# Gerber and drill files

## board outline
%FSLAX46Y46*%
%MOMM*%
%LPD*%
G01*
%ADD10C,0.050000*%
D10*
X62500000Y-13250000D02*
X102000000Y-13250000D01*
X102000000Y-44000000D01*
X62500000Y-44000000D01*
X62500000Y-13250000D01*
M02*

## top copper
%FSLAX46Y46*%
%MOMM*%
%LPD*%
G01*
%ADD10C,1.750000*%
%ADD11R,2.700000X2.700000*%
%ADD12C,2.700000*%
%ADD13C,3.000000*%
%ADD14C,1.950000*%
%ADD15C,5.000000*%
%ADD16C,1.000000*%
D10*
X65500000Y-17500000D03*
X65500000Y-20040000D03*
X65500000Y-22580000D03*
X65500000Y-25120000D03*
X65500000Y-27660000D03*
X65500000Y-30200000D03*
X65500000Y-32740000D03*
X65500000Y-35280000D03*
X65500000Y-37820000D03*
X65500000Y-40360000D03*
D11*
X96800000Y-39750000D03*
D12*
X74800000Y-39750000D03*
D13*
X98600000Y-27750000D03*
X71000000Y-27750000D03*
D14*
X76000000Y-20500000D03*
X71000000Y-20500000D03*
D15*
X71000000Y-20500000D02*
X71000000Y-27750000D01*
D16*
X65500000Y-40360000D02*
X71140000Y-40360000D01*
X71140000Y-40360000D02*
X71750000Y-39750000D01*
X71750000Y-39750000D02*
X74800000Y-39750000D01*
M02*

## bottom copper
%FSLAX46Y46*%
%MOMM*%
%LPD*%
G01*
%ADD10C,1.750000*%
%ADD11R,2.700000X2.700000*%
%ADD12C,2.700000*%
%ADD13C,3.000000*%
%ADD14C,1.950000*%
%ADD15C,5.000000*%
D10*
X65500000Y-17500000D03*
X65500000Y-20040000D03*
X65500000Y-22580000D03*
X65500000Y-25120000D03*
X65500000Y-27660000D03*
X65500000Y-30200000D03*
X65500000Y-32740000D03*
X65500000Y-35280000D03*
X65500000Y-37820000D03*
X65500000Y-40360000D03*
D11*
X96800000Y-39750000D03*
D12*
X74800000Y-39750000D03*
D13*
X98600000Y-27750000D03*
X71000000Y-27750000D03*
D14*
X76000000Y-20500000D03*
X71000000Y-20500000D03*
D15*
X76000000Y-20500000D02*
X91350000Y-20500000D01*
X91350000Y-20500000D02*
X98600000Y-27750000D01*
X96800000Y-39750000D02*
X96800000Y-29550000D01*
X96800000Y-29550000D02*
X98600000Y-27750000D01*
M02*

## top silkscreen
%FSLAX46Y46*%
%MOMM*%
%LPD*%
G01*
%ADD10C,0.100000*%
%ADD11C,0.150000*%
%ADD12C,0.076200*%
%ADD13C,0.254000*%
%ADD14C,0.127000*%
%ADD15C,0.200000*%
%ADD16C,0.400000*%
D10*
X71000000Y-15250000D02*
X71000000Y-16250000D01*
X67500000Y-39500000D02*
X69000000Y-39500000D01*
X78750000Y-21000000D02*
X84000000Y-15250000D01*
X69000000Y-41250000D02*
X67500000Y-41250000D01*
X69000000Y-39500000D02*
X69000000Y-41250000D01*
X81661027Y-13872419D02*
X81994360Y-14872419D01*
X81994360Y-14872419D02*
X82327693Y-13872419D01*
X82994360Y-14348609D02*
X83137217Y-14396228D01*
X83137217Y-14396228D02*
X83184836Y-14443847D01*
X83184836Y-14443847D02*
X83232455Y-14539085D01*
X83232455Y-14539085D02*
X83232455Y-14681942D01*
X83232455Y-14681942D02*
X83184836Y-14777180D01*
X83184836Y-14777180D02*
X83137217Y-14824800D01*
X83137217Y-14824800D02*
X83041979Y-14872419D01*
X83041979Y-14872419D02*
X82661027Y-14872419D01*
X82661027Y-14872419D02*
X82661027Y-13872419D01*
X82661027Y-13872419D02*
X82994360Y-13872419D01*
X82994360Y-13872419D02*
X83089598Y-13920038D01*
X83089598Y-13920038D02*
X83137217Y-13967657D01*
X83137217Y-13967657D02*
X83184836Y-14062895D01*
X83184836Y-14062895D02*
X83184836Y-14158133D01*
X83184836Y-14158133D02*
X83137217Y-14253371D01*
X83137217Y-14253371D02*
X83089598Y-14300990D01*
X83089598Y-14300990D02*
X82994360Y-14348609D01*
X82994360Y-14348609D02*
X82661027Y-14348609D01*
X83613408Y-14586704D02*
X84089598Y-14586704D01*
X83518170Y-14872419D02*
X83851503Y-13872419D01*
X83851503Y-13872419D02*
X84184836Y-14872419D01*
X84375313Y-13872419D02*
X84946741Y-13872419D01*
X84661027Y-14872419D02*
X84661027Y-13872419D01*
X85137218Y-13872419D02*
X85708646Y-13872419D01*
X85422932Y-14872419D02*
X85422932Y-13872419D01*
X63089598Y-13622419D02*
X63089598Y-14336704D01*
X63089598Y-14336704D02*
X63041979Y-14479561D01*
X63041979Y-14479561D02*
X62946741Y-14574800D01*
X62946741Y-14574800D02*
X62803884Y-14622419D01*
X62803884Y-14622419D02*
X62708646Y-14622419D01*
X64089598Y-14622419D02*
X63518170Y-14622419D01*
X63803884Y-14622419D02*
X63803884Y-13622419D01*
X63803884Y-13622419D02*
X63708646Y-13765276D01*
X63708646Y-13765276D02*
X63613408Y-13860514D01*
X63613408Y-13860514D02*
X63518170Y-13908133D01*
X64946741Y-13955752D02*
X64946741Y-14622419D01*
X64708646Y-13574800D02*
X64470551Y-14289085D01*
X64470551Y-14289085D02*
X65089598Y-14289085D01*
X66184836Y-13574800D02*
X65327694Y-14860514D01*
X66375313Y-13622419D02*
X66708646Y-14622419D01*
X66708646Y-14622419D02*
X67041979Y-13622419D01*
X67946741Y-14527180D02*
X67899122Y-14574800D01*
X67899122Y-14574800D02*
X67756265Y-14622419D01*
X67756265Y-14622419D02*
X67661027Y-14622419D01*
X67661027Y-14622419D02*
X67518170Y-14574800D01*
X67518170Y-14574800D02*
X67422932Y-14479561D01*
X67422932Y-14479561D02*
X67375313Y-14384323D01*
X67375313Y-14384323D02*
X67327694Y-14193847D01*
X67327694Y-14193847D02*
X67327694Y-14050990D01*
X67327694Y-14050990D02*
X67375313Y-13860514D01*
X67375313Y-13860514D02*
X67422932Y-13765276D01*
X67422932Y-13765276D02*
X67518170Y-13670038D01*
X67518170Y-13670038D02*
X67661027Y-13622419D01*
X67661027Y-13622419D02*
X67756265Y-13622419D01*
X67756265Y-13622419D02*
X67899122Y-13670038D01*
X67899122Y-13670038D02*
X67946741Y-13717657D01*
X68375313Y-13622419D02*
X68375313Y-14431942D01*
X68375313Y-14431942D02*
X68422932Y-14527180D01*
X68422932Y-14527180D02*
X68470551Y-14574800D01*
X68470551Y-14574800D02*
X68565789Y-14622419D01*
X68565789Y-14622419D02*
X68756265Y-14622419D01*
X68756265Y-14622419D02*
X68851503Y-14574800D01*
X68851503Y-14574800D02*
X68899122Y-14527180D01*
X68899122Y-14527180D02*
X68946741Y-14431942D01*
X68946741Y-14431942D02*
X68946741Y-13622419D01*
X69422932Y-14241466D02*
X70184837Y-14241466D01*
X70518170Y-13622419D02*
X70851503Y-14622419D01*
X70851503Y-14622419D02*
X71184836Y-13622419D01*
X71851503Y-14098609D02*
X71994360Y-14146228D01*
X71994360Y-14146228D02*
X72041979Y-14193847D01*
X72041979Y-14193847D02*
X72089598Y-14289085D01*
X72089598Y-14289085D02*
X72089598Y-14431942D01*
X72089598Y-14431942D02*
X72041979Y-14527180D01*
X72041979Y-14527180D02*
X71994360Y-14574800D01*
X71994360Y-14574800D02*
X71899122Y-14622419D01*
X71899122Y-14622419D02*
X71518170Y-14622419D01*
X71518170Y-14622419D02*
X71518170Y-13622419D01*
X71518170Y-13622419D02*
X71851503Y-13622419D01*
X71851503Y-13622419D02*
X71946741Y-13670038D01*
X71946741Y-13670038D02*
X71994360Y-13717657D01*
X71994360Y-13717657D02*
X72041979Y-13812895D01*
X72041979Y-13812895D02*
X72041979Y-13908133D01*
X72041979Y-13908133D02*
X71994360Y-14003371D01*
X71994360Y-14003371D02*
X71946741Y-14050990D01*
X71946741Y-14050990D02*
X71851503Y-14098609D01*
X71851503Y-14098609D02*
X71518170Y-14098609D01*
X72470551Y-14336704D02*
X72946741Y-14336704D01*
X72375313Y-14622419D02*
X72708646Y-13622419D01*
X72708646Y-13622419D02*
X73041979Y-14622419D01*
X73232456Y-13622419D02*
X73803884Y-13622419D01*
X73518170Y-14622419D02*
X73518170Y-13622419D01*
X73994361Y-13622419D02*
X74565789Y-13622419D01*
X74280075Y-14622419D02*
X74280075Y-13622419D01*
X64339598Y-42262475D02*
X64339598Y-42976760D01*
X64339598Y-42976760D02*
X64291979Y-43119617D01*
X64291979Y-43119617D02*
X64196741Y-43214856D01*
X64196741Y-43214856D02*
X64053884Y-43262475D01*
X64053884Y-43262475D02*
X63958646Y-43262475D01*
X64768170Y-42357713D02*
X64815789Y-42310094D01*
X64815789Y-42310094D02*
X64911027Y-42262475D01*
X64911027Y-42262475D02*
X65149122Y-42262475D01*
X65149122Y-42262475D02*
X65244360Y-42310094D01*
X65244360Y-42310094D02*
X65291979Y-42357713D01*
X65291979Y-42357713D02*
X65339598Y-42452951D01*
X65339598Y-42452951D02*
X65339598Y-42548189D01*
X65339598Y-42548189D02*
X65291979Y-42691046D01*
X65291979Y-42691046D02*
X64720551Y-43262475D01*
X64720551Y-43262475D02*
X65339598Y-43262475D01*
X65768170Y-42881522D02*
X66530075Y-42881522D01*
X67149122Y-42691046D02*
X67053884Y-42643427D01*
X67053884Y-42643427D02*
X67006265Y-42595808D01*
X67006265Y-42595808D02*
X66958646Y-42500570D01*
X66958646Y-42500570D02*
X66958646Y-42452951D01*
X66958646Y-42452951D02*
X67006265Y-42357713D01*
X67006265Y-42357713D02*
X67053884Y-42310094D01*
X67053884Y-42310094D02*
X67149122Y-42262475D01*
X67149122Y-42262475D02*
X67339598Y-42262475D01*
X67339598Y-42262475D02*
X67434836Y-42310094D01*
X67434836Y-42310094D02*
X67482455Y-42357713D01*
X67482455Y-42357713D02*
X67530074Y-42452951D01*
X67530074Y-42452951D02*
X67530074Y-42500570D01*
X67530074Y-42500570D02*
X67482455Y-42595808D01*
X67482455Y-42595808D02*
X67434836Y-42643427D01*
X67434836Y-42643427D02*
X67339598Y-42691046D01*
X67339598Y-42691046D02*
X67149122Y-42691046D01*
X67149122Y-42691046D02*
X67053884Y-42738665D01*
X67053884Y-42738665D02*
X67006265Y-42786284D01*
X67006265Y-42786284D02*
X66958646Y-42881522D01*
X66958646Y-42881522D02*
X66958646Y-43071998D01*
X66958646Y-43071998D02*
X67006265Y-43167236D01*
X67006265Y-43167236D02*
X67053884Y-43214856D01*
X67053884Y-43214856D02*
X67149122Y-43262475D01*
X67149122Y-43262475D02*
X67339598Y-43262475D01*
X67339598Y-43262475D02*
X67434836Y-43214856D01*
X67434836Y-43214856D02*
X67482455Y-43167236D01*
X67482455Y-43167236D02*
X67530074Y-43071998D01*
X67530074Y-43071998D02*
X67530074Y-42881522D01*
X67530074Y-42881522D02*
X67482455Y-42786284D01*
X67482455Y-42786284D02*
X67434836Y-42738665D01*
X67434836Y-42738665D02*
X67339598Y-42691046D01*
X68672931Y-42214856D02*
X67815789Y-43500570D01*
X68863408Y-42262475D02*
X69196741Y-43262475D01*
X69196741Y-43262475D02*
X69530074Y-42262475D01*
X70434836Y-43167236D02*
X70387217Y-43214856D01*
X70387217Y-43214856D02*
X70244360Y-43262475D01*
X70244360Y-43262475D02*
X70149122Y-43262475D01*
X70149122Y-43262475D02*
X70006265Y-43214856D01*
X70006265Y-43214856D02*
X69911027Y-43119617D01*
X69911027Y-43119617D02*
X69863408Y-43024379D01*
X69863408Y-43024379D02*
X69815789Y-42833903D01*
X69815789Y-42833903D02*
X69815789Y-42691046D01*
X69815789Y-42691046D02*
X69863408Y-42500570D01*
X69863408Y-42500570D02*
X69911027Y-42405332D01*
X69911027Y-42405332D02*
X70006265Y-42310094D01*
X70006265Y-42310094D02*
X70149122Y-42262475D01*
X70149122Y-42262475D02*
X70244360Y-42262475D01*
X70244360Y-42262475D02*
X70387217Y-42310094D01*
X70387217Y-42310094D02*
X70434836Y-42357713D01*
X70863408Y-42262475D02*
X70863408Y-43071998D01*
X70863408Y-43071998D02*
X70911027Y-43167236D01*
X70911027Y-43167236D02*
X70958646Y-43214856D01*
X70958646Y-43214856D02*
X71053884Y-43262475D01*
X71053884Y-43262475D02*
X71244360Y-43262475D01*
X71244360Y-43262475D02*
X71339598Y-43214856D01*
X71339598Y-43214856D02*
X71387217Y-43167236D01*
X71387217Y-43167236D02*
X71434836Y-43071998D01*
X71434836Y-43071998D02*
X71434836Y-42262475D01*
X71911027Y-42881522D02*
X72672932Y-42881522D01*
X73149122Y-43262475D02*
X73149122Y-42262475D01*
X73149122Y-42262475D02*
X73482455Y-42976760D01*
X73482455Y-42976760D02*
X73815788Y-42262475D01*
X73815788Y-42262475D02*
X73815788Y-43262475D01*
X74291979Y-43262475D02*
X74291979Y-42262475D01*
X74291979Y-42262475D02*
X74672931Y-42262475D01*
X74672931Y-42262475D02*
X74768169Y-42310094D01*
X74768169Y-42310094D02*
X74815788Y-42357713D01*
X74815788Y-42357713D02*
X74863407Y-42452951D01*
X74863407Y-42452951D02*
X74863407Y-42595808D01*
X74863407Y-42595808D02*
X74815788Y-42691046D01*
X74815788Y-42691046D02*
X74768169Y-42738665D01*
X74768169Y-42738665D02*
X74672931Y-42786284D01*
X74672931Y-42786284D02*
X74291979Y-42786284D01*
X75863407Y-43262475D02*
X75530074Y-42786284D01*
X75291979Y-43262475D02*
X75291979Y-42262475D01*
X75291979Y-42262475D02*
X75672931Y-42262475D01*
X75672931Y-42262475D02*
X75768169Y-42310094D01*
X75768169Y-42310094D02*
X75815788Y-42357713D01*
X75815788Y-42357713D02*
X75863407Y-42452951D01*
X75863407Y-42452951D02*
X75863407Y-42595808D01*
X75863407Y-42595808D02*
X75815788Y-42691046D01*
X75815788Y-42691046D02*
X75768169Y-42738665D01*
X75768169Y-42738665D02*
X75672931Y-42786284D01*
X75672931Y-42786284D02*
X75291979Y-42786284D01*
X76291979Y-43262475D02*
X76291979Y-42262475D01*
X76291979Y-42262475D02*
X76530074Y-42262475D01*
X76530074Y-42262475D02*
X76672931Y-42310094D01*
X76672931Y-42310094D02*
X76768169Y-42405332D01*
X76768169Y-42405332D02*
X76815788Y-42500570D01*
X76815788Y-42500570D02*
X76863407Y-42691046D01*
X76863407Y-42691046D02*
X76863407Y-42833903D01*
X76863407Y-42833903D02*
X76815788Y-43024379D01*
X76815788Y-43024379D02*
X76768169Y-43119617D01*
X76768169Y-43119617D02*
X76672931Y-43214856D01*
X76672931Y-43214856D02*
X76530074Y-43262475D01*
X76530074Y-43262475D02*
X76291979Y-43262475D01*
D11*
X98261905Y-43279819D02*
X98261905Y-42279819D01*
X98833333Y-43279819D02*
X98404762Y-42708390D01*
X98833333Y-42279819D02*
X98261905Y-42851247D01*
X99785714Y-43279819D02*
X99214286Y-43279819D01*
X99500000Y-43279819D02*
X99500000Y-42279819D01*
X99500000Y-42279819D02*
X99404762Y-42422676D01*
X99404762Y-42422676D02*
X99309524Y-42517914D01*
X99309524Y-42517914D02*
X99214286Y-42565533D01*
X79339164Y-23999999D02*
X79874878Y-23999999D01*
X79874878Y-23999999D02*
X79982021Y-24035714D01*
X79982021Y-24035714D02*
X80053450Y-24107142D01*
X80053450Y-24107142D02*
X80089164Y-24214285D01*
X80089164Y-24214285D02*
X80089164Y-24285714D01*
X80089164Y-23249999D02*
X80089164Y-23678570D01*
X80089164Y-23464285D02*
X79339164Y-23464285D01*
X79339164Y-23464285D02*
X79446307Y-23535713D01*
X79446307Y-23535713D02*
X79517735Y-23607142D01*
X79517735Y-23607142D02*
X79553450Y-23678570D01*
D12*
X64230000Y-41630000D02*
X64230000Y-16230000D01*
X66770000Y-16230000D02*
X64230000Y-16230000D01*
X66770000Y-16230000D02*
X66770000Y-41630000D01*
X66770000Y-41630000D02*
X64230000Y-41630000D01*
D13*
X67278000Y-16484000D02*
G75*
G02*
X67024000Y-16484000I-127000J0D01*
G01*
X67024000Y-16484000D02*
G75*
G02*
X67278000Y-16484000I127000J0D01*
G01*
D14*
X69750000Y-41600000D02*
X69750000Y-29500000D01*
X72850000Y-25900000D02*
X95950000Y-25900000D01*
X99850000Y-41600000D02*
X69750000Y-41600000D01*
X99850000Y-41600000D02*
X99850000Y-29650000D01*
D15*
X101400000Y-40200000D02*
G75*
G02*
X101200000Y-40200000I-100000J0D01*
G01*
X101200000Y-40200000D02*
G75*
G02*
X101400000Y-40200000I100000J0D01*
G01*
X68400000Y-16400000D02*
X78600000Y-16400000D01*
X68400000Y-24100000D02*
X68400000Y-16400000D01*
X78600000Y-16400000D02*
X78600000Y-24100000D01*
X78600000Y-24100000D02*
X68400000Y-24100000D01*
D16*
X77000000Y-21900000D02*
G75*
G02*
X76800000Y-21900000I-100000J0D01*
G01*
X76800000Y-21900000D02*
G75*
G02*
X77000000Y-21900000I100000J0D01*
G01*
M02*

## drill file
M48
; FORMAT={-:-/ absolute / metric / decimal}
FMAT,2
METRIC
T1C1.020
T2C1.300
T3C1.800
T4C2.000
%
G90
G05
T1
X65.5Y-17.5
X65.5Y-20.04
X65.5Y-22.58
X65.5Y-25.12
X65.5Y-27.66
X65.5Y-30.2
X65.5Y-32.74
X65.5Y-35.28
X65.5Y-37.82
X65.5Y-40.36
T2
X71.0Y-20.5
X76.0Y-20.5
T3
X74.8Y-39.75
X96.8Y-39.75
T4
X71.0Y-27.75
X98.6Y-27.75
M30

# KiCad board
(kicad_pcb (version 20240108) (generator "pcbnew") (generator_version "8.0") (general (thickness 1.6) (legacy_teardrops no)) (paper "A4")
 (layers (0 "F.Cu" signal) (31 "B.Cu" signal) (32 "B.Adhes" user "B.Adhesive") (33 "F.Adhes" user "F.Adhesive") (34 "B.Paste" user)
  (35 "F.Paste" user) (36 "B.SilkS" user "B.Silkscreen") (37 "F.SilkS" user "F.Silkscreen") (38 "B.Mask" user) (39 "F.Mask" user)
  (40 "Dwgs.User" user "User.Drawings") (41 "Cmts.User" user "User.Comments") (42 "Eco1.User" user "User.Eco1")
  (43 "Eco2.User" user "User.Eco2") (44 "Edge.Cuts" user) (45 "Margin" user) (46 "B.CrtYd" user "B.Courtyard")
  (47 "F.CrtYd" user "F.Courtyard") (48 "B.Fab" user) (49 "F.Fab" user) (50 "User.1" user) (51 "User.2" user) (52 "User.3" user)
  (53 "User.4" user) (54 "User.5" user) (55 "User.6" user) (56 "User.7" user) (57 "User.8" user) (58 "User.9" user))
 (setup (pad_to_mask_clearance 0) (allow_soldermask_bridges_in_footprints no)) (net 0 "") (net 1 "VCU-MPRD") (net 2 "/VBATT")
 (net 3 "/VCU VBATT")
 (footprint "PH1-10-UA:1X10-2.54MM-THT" (layer "F.Cu") (at 65.5 17.5 -90)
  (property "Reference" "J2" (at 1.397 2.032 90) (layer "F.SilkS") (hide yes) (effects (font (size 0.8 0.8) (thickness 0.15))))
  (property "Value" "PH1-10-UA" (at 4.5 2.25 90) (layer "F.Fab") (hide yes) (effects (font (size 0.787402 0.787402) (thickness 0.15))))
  (fp_line (start 24.13 1.27) (end -1.27 1.27) (stroke (width 0.0762) (type solid)) (layer "F.SilkS"))
  (fp_line (start -1.27 -1.27) (end -1.27 1.27) (stroke (width 0.0762) (type solid)) (layer "F.SilkS"))
  (fp_line (start -1.27 -1.27) (end 24.13 -1.27) (stroke (width 0.0762) (type solid)) (layer "F.SilkS"))
  (fp_line (start 24.13 -1.27) (end 24.13 1.27) (stroke (width 0.0762) (type solid)) (layer "F.SilkS"))
  (fp_circle (center -1.016 -1.651) (end -0.762 -1.651) (stroke (width 0) (type solid)) (fill solid) (layer "F.SilkS"))
  (pad "1" thru_hole circle (at 0 0 270) (size 1.75 1.75) (drill 1.02) (layers "*.Cu" "*.Mask") (remove_unused_layers no)
   (solder_mask_margin 0.102))
  (pad "2" thru_hole circle (at 2.54 0 270) (size 1.75 1.75) (drill 1.02) (layers "*.Cu" "*.Mask") (remove_unused_layers no)
   (solder_mask_margin 0.102))
  (pad "3" thru_hole circle (at 5.08 0 270) (size 1.75 1.75) (drill 1.02) (layers "*.Cu" "*.Mask") (remove_unused_layers no)
   (solder_mask_margin 0.102))
  (pad "4" thru_hole circle (at 7.62 0 270) (size 1.75 1.75) (drill 1.02) (layers "*.Cu" "*.Mask") (remove_unused_layers no)
   (solder_mask_margin 0.102))
  (pad "5" thru_hole circle (at 10.16 0 270) (size 1.75 1.75) (drill 1.02) (layers "*.Cu" "*.Mask") (remove_unused_layers no)
   (solder_mask_margin 0.102))
  (pad "6" thru_hole circle (at 12.7 0 270) (size 1.75 1.75) (drill 1.02) (layers "*.Cu" "*.Mask") (remove_unused_layers no)
   (solder_mask_margin 0.102))
  (pad "7" thru_hole circle (at 15.24 0 270) (size 1.75 1.75) (drill 1.02) (layers "*.Cu" "*.Mask") (remove_unused_layers no)
   (solder_mask_margin 0.102))
  (pad "8" thru_hole circle (at 17.78 0 270) (size 1.75 1.75) (drill 1.02) (layers "*.Cu" "*.Mask") (remove_unused_layers no)
   (solder_mask_margin 0.102))
  (pad "9" thru_hole circle (at 20.32 0 270) (size 1.75 1.75) (drill 1.02) (layers "*.Cu" "*.Mask") (remove_unused_layers no)
   (solder_mask_margin 0.102))
  (pad "10" thru_hole circle (at 22.86 0 270) (size 1.75 1.75) (drill 1.02) (layers "*.Cu" "*.Mask") (remove_unused_layers no)
   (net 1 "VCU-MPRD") (solder_mask_margin 0.102)))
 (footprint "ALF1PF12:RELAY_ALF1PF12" (layer "F.Cu") (at 84.8 33.75 180)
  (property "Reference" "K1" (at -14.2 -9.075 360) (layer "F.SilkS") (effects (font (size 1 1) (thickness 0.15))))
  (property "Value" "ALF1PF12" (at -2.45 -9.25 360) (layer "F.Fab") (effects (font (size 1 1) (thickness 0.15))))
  (fp_line (start 15.05 -7.85) (end 15.05 4.25) (stroke (width 0.127) (type solid)) (layer "F.SilkS"))
  (fp_line (start 11.95 7.85) (end -11.15 7.85) (stroke (width 0.127) (type solid)) (layer "F.SilkS"))
  (fp_line (start -15.05 -7.85) (end 15.05 -7.85) (stroke (width 0.127) (type solid)) (layer "F.SilkS"))
  (fp_line (start -15.05 -7.85) (end -15.05 4.1) (stroke (width 0.127) (type solid)) (layer "F.SilkS"))
  (fp_circle (center -16.5 -6.45) (end -16.4 -6.45) (stroke (width 0.2) (type solid)) (fill none) (layer "F.SilkS"))
  (pad "1" thru_hole rect (at -12 -6 180) (size 2.7 2.7) (drill 1.8) (layers "*.Cu" "*.Mask") (remove_unused_layers no) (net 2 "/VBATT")
   (solder_mask_margin 0.102))
  (pad "2" thru_hole circle (at 10 -6 180) (size 2.7 2.7) (drill 1.8) (layers "*.Cu" "*.Mask") (remove_unused_layers no) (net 1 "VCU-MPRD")
   (solder_mask_margin 0.102))
  (pad "3" thru_hole circle (at -13.8 6 180) (size 3 3) (drill 2) (layers "*.Cu" "*.Mask") (remove_unused_layers no) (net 2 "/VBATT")
   (solder_mask_margin 0.102))
  (pad "4" thru_hole circle (at 13.8 6 180) (size 3 3) (drill 2) (layers "*.Cu" "*.Mask") (remove_unused_layers no) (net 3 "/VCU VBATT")
   (solder_mask_margin 0.102)))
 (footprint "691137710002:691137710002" (layer "F.Cu") (at 73.5 20.5 180)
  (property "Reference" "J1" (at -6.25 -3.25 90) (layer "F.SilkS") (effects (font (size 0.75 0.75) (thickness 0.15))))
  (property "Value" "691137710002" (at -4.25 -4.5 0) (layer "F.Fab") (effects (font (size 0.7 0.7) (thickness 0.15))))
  (fp_line (start 5.1 4.1) (end -5.1 4.1) (stroke (width 0.2) (type solid)) (layer "F.SilkS"))
  (fp_line (start 5.1 -3.6) (end 5.1 4.1) (stroke (width 0.2) (type solid)) (layer "F.SilkS"))
  (fp_line (start -5.1 4.1) (end -5.1 -3.6) (stroke (width 0.2) (type solid)) (layer "F.SilkS"))
  (fp_line (start -5.1 -3.6) (end 5.1 -3.6) (stroke (width 0.2) (type solid)) (layer "F.SilkS"))
  (fp_circle (center -3.4 -1.4) (end -3.3 -1.4) (stroke (width 0.4) (type solid)) (fill none) (layer "F.SilkS"))
  (pad "1" thru_hole circle (at -2.5 0 180) (size 1.95 1.95) (drill 1.3) (layers "*.Cu" "*.Mask") (remove_unused_layers no) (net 2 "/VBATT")
   (solder_mask_margin 0.102))
  (pad "2" thru_hole circle (at 2.5 0 180) (size 1.95 1.95) (drill 1.3) (layers "*.Cu" "*.Mask") (remove_unused_layers no)
   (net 3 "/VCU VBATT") (solder_mask_margin 0.102)))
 (gr_line (start 71 15.25) (end 71 16.25) (stroke (width 0.1) (type default)) (layer "F.SilkS"))
 (gr_line (start 67.5 39.5) (end 69 39.5) (stroke (width 0.1) (type default)) (layer "F.SilkS"))
 (gr_line (start 78.75 21) (end 84 15.25) (stroke (width 0.1) (type default)) (layer "F.SilkS"))
 (gr_line (start 69 41.25) (end 67.5 41.25) (stroke (width 0.1) (type default)) (layer "F.SilkS"))
 (gr_line (start 69 39.5) (end 69 41.25) (stroke (width 0.1) (type default)) (layer "F.SilkS"))
 (gr_rect (start 62.5 13.25) (end 102 44) (stroke (width 0.05) (type default)) (fill none) (layer "Edge.Cuts"))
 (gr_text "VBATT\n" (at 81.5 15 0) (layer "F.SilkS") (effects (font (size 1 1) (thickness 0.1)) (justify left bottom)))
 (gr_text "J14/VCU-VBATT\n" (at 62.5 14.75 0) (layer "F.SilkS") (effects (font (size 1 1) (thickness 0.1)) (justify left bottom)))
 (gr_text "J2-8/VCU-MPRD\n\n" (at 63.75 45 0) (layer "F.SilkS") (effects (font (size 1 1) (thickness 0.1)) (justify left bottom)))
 (segment (start 76 20.5) (end 91.35 20.5) (width 5) (layer "B.Cu") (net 2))
 (segment (start 91.35 20.5) (end 98.6 27.75) (width 5) (layer "B.Cu") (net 2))
 (segment (start 96.8 39.75) (end 96.8 29.55) (width 5) (layer "B.Cu") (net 2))
 (segment (start 96.8 29.55) (end 98.6 27.75) (width 5) (layer "B.Cu") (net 2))
 (segment (start 71 20.5) (end 71 27.75) (width 5) (layer "F.Cu") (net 3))
 (segment (start 65.5 40.36) (end 71.14 40.36) (width 1) (layer "F.Cu") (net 1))
 (segment (start 71.14 40.36) (end 71.75 39.75) (width 1) (layer "F.Cu") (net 1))
 (segment (start 71.75 39.75) (end 74.8 39.75) (width 1) (layer "F.Cu") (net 1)))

